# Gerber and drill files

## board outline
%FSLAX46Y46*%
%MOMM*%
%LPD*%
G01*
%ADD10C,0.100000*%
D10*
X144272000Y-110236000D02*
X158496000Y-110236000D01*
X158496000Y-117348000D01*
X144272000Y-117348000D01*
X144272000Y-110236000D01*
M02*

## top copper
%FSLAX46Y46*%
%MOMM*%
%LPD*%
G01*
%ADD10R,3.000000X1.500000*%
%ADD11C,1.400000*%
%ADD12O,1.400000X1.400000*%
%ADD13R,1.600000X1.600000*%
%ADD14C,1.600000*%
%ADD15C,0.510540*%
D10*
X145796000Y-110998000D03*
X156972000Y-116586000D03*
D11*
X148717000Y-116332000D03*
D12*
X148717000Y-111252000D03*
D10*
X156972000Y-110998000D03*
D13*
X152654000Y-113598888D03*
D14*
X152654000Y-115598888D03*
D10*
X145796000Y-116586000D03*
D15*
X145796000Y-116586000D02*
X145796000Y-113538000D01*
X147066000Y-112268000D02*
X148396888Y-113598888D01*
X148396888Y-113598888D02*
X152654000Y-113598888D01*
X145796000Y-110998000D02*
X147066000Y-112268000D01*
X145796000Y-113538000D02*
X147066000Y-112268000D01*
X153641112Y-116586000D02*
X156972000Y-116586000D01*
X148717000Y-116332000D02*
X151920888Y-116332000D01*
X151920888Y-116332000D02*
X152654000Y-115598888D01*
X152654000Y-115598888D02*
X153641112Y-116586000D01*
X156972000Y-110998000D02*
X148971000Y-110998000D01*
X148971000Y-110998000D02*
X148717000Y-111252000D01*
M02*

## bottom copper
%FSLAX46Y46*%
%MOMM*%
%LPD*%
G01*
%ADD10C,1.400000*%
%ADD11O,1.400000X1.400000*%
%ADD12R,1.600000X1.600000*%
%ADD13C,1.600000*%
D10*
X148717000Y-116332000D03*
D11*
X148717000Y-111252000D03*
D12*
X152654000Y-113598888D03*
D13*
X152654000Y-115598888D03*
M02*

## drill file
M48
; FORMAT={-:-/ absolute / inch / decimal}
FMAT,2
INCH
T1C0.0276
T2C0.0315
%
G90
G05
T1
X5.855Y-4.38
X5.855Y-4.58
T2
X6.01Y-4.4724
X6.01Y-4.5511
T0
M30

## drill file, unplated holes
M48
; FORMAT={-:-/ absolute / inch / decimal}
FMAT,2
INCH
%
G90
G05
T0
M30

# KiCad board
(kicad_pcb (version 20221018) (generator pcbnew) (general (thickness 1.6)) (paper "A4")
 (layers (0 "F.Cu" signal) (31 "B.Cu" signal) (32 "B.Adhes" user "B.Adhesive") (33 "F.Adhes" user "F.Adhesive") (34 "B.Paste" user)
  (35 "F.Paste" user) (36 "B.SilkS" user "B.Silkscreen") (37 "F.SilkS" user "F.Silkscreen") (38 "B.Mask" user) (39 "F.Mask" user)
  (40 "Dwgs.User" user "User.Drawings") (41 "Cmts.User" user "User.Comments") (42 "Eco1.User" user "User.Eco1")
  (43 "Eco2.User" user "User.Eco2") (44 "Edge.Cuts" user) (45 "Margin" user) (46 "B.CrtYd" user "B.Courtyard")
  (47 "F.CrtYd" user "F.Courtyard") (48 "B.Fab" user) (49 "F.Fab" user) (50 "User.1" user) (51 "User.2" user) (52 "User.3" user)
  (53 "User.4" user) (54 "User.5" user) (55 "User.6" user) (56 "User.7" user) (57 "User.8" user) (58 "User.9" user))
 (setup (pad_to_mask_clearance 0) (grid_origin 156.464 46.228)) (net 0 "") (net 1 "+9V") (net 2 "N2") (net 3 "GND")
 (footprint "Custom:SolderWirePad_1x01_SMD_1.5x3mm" (layer "F.Cu") (at 145.796 110.998 90)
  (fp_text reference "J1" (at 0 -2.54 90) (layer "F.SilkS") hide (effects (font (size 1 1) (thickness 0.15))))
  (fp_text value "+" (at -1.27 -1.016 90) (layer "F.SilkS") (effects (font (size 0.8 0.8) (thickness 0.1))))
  (pad "1" smd rect (at 0 0 90) (size 1.5 3) (layers "F.Cu" "F.Paste" "F.Mask") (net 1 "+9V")))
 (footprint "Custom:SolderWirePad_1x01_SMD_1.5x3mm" (layer "F.Cu") (at 156.972 116.586 90)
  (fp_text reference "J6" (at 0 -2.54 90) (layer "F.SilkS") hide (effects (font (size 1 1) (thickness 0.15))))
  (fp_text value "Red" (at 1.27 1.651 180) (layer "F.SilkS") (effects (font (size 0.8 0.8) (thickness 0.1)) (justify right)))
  (pad "1" smd rect (at 0 0 90) (size 1.5 3) (layers "F.Cu" "F.Paste" "F.Mask") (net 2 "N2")))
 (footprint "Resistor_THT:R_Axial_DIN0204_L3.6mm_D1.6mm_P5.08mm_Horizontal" (layer "F.Cu") (at 148.717 116.332 90)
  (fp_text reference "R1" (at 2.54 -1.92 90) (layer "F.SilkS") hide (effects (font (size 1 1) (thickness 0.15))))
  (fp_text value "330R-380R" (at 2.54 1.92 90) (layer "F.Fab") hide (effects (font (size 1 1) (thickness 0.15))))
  (pad "1" thru_hole circle (at 0 0 90) (size 1.4 1.4) (drill 0.7) (layers "*.Cu" "*.Mask") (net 2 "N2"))
  (pad "2" thru_hole oval (at 5.08 0 90) (size 1.4 1.4) (drill 0.7) (layers "*.Cu" "*.Mask") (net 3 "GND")))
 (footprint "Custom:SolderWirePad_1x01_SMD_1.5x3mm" (layer "F.Cu") (at 156.972 110.998 90)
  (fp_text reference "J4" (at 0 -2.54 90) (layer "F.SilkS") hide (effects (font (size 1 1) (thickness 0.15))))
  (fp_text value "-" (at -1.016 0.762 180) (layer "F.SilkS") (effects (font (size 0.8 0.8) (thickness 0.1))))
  (pad "1" smd rect (at 0 0 90) (size 1.5 3) (layers "F.Cu" "F.Paste" "F.Mask") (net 3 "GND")))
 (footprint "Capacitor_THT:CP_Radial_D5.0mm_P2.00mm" (layer "F.Cu") (at 152.654 113.598888 -90)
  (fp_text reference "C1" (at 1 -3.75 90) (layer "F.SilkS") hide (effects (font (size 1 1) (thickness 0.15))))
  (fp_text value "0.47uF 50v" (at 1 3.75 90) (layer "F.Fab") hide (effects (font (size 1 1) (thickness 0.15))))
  (pad "1" thru_hole rect (at 0 0 270) (size 1.6 1.6) (drill 0.8) (layers "*.Cu" "*.Mask") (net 1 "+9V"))
  (pad "2" thru_hole circle (at 2 0 270) (size 1.6 1.6) (drill 0.8) (layers "*.Cu" "*.Mask") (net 2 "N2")))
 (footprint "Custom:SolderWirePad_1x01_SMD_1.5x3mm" (layer "F.Cu") (at 145.796 116.586 90)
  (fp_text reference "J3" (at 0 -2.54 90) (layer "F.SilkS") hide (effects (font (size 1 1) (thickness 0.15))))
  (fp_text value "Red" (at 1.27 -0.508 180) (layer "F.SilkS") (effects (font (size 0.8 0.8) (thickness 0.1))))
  (pad "1" smd rect (at 0 0 90) (size 1.5 3) (layers "F.Cu" "F.Paste" "F.Mask") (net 1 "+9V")))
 (gr_rect (start 144.272 110.236) (end 158.496 117.348) (stroke (width 0.1) (type default)) (fill none) (layer "Edge.Cuts"))
 (segment (start 145.796 116.586) (end 145.796 113.538) (width 0.51054) (layer "F.Cu") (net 1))
 (segment (start 147.066 112.268) (end 148.396888 113.598888) (width 0.51054) (layer "F.Cu") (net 1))
 (segment (start 148.396888 113.598888) (end 152.654 113.598888) (width 0.51054) (layer "F.Cu") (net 1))
 (segment (start 145.796 110.998) (end 147.066 112.268) (width 0.51054) (layer "F.Cu") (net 1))
 (segment (start 145.796 113.538) (end 147.066 112.268) (width 0.51054) (layer "F.Cu") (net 1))
 (segment (start 153.641112 116.586) (end 156.972 116.586) (width 0.51054) (layer "F.Cu") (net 2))
 (segment (start 148.717 116.332) (end 151.920888 116.332) (width 0.51054) (layer "F.Cu") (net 2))
 (segment (start 151.920888 116.332) (end 152.654 115.598888) (width 0.51054) (layer "F.Cu") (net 2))
 (segment (start 152.654 115.598888) (end 153.641112 116.586) (width 0.51054) (layer "F.Cu") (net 2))
 (segment (start 156.972 110.998) (end 148.971 110.998) (width 0.51054) (layer "F.Cu") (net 3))
 (segment (start 148.971 110.998) (end 148.717 111.252) (width 0.51054) (layer "F.Cu") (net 3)))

